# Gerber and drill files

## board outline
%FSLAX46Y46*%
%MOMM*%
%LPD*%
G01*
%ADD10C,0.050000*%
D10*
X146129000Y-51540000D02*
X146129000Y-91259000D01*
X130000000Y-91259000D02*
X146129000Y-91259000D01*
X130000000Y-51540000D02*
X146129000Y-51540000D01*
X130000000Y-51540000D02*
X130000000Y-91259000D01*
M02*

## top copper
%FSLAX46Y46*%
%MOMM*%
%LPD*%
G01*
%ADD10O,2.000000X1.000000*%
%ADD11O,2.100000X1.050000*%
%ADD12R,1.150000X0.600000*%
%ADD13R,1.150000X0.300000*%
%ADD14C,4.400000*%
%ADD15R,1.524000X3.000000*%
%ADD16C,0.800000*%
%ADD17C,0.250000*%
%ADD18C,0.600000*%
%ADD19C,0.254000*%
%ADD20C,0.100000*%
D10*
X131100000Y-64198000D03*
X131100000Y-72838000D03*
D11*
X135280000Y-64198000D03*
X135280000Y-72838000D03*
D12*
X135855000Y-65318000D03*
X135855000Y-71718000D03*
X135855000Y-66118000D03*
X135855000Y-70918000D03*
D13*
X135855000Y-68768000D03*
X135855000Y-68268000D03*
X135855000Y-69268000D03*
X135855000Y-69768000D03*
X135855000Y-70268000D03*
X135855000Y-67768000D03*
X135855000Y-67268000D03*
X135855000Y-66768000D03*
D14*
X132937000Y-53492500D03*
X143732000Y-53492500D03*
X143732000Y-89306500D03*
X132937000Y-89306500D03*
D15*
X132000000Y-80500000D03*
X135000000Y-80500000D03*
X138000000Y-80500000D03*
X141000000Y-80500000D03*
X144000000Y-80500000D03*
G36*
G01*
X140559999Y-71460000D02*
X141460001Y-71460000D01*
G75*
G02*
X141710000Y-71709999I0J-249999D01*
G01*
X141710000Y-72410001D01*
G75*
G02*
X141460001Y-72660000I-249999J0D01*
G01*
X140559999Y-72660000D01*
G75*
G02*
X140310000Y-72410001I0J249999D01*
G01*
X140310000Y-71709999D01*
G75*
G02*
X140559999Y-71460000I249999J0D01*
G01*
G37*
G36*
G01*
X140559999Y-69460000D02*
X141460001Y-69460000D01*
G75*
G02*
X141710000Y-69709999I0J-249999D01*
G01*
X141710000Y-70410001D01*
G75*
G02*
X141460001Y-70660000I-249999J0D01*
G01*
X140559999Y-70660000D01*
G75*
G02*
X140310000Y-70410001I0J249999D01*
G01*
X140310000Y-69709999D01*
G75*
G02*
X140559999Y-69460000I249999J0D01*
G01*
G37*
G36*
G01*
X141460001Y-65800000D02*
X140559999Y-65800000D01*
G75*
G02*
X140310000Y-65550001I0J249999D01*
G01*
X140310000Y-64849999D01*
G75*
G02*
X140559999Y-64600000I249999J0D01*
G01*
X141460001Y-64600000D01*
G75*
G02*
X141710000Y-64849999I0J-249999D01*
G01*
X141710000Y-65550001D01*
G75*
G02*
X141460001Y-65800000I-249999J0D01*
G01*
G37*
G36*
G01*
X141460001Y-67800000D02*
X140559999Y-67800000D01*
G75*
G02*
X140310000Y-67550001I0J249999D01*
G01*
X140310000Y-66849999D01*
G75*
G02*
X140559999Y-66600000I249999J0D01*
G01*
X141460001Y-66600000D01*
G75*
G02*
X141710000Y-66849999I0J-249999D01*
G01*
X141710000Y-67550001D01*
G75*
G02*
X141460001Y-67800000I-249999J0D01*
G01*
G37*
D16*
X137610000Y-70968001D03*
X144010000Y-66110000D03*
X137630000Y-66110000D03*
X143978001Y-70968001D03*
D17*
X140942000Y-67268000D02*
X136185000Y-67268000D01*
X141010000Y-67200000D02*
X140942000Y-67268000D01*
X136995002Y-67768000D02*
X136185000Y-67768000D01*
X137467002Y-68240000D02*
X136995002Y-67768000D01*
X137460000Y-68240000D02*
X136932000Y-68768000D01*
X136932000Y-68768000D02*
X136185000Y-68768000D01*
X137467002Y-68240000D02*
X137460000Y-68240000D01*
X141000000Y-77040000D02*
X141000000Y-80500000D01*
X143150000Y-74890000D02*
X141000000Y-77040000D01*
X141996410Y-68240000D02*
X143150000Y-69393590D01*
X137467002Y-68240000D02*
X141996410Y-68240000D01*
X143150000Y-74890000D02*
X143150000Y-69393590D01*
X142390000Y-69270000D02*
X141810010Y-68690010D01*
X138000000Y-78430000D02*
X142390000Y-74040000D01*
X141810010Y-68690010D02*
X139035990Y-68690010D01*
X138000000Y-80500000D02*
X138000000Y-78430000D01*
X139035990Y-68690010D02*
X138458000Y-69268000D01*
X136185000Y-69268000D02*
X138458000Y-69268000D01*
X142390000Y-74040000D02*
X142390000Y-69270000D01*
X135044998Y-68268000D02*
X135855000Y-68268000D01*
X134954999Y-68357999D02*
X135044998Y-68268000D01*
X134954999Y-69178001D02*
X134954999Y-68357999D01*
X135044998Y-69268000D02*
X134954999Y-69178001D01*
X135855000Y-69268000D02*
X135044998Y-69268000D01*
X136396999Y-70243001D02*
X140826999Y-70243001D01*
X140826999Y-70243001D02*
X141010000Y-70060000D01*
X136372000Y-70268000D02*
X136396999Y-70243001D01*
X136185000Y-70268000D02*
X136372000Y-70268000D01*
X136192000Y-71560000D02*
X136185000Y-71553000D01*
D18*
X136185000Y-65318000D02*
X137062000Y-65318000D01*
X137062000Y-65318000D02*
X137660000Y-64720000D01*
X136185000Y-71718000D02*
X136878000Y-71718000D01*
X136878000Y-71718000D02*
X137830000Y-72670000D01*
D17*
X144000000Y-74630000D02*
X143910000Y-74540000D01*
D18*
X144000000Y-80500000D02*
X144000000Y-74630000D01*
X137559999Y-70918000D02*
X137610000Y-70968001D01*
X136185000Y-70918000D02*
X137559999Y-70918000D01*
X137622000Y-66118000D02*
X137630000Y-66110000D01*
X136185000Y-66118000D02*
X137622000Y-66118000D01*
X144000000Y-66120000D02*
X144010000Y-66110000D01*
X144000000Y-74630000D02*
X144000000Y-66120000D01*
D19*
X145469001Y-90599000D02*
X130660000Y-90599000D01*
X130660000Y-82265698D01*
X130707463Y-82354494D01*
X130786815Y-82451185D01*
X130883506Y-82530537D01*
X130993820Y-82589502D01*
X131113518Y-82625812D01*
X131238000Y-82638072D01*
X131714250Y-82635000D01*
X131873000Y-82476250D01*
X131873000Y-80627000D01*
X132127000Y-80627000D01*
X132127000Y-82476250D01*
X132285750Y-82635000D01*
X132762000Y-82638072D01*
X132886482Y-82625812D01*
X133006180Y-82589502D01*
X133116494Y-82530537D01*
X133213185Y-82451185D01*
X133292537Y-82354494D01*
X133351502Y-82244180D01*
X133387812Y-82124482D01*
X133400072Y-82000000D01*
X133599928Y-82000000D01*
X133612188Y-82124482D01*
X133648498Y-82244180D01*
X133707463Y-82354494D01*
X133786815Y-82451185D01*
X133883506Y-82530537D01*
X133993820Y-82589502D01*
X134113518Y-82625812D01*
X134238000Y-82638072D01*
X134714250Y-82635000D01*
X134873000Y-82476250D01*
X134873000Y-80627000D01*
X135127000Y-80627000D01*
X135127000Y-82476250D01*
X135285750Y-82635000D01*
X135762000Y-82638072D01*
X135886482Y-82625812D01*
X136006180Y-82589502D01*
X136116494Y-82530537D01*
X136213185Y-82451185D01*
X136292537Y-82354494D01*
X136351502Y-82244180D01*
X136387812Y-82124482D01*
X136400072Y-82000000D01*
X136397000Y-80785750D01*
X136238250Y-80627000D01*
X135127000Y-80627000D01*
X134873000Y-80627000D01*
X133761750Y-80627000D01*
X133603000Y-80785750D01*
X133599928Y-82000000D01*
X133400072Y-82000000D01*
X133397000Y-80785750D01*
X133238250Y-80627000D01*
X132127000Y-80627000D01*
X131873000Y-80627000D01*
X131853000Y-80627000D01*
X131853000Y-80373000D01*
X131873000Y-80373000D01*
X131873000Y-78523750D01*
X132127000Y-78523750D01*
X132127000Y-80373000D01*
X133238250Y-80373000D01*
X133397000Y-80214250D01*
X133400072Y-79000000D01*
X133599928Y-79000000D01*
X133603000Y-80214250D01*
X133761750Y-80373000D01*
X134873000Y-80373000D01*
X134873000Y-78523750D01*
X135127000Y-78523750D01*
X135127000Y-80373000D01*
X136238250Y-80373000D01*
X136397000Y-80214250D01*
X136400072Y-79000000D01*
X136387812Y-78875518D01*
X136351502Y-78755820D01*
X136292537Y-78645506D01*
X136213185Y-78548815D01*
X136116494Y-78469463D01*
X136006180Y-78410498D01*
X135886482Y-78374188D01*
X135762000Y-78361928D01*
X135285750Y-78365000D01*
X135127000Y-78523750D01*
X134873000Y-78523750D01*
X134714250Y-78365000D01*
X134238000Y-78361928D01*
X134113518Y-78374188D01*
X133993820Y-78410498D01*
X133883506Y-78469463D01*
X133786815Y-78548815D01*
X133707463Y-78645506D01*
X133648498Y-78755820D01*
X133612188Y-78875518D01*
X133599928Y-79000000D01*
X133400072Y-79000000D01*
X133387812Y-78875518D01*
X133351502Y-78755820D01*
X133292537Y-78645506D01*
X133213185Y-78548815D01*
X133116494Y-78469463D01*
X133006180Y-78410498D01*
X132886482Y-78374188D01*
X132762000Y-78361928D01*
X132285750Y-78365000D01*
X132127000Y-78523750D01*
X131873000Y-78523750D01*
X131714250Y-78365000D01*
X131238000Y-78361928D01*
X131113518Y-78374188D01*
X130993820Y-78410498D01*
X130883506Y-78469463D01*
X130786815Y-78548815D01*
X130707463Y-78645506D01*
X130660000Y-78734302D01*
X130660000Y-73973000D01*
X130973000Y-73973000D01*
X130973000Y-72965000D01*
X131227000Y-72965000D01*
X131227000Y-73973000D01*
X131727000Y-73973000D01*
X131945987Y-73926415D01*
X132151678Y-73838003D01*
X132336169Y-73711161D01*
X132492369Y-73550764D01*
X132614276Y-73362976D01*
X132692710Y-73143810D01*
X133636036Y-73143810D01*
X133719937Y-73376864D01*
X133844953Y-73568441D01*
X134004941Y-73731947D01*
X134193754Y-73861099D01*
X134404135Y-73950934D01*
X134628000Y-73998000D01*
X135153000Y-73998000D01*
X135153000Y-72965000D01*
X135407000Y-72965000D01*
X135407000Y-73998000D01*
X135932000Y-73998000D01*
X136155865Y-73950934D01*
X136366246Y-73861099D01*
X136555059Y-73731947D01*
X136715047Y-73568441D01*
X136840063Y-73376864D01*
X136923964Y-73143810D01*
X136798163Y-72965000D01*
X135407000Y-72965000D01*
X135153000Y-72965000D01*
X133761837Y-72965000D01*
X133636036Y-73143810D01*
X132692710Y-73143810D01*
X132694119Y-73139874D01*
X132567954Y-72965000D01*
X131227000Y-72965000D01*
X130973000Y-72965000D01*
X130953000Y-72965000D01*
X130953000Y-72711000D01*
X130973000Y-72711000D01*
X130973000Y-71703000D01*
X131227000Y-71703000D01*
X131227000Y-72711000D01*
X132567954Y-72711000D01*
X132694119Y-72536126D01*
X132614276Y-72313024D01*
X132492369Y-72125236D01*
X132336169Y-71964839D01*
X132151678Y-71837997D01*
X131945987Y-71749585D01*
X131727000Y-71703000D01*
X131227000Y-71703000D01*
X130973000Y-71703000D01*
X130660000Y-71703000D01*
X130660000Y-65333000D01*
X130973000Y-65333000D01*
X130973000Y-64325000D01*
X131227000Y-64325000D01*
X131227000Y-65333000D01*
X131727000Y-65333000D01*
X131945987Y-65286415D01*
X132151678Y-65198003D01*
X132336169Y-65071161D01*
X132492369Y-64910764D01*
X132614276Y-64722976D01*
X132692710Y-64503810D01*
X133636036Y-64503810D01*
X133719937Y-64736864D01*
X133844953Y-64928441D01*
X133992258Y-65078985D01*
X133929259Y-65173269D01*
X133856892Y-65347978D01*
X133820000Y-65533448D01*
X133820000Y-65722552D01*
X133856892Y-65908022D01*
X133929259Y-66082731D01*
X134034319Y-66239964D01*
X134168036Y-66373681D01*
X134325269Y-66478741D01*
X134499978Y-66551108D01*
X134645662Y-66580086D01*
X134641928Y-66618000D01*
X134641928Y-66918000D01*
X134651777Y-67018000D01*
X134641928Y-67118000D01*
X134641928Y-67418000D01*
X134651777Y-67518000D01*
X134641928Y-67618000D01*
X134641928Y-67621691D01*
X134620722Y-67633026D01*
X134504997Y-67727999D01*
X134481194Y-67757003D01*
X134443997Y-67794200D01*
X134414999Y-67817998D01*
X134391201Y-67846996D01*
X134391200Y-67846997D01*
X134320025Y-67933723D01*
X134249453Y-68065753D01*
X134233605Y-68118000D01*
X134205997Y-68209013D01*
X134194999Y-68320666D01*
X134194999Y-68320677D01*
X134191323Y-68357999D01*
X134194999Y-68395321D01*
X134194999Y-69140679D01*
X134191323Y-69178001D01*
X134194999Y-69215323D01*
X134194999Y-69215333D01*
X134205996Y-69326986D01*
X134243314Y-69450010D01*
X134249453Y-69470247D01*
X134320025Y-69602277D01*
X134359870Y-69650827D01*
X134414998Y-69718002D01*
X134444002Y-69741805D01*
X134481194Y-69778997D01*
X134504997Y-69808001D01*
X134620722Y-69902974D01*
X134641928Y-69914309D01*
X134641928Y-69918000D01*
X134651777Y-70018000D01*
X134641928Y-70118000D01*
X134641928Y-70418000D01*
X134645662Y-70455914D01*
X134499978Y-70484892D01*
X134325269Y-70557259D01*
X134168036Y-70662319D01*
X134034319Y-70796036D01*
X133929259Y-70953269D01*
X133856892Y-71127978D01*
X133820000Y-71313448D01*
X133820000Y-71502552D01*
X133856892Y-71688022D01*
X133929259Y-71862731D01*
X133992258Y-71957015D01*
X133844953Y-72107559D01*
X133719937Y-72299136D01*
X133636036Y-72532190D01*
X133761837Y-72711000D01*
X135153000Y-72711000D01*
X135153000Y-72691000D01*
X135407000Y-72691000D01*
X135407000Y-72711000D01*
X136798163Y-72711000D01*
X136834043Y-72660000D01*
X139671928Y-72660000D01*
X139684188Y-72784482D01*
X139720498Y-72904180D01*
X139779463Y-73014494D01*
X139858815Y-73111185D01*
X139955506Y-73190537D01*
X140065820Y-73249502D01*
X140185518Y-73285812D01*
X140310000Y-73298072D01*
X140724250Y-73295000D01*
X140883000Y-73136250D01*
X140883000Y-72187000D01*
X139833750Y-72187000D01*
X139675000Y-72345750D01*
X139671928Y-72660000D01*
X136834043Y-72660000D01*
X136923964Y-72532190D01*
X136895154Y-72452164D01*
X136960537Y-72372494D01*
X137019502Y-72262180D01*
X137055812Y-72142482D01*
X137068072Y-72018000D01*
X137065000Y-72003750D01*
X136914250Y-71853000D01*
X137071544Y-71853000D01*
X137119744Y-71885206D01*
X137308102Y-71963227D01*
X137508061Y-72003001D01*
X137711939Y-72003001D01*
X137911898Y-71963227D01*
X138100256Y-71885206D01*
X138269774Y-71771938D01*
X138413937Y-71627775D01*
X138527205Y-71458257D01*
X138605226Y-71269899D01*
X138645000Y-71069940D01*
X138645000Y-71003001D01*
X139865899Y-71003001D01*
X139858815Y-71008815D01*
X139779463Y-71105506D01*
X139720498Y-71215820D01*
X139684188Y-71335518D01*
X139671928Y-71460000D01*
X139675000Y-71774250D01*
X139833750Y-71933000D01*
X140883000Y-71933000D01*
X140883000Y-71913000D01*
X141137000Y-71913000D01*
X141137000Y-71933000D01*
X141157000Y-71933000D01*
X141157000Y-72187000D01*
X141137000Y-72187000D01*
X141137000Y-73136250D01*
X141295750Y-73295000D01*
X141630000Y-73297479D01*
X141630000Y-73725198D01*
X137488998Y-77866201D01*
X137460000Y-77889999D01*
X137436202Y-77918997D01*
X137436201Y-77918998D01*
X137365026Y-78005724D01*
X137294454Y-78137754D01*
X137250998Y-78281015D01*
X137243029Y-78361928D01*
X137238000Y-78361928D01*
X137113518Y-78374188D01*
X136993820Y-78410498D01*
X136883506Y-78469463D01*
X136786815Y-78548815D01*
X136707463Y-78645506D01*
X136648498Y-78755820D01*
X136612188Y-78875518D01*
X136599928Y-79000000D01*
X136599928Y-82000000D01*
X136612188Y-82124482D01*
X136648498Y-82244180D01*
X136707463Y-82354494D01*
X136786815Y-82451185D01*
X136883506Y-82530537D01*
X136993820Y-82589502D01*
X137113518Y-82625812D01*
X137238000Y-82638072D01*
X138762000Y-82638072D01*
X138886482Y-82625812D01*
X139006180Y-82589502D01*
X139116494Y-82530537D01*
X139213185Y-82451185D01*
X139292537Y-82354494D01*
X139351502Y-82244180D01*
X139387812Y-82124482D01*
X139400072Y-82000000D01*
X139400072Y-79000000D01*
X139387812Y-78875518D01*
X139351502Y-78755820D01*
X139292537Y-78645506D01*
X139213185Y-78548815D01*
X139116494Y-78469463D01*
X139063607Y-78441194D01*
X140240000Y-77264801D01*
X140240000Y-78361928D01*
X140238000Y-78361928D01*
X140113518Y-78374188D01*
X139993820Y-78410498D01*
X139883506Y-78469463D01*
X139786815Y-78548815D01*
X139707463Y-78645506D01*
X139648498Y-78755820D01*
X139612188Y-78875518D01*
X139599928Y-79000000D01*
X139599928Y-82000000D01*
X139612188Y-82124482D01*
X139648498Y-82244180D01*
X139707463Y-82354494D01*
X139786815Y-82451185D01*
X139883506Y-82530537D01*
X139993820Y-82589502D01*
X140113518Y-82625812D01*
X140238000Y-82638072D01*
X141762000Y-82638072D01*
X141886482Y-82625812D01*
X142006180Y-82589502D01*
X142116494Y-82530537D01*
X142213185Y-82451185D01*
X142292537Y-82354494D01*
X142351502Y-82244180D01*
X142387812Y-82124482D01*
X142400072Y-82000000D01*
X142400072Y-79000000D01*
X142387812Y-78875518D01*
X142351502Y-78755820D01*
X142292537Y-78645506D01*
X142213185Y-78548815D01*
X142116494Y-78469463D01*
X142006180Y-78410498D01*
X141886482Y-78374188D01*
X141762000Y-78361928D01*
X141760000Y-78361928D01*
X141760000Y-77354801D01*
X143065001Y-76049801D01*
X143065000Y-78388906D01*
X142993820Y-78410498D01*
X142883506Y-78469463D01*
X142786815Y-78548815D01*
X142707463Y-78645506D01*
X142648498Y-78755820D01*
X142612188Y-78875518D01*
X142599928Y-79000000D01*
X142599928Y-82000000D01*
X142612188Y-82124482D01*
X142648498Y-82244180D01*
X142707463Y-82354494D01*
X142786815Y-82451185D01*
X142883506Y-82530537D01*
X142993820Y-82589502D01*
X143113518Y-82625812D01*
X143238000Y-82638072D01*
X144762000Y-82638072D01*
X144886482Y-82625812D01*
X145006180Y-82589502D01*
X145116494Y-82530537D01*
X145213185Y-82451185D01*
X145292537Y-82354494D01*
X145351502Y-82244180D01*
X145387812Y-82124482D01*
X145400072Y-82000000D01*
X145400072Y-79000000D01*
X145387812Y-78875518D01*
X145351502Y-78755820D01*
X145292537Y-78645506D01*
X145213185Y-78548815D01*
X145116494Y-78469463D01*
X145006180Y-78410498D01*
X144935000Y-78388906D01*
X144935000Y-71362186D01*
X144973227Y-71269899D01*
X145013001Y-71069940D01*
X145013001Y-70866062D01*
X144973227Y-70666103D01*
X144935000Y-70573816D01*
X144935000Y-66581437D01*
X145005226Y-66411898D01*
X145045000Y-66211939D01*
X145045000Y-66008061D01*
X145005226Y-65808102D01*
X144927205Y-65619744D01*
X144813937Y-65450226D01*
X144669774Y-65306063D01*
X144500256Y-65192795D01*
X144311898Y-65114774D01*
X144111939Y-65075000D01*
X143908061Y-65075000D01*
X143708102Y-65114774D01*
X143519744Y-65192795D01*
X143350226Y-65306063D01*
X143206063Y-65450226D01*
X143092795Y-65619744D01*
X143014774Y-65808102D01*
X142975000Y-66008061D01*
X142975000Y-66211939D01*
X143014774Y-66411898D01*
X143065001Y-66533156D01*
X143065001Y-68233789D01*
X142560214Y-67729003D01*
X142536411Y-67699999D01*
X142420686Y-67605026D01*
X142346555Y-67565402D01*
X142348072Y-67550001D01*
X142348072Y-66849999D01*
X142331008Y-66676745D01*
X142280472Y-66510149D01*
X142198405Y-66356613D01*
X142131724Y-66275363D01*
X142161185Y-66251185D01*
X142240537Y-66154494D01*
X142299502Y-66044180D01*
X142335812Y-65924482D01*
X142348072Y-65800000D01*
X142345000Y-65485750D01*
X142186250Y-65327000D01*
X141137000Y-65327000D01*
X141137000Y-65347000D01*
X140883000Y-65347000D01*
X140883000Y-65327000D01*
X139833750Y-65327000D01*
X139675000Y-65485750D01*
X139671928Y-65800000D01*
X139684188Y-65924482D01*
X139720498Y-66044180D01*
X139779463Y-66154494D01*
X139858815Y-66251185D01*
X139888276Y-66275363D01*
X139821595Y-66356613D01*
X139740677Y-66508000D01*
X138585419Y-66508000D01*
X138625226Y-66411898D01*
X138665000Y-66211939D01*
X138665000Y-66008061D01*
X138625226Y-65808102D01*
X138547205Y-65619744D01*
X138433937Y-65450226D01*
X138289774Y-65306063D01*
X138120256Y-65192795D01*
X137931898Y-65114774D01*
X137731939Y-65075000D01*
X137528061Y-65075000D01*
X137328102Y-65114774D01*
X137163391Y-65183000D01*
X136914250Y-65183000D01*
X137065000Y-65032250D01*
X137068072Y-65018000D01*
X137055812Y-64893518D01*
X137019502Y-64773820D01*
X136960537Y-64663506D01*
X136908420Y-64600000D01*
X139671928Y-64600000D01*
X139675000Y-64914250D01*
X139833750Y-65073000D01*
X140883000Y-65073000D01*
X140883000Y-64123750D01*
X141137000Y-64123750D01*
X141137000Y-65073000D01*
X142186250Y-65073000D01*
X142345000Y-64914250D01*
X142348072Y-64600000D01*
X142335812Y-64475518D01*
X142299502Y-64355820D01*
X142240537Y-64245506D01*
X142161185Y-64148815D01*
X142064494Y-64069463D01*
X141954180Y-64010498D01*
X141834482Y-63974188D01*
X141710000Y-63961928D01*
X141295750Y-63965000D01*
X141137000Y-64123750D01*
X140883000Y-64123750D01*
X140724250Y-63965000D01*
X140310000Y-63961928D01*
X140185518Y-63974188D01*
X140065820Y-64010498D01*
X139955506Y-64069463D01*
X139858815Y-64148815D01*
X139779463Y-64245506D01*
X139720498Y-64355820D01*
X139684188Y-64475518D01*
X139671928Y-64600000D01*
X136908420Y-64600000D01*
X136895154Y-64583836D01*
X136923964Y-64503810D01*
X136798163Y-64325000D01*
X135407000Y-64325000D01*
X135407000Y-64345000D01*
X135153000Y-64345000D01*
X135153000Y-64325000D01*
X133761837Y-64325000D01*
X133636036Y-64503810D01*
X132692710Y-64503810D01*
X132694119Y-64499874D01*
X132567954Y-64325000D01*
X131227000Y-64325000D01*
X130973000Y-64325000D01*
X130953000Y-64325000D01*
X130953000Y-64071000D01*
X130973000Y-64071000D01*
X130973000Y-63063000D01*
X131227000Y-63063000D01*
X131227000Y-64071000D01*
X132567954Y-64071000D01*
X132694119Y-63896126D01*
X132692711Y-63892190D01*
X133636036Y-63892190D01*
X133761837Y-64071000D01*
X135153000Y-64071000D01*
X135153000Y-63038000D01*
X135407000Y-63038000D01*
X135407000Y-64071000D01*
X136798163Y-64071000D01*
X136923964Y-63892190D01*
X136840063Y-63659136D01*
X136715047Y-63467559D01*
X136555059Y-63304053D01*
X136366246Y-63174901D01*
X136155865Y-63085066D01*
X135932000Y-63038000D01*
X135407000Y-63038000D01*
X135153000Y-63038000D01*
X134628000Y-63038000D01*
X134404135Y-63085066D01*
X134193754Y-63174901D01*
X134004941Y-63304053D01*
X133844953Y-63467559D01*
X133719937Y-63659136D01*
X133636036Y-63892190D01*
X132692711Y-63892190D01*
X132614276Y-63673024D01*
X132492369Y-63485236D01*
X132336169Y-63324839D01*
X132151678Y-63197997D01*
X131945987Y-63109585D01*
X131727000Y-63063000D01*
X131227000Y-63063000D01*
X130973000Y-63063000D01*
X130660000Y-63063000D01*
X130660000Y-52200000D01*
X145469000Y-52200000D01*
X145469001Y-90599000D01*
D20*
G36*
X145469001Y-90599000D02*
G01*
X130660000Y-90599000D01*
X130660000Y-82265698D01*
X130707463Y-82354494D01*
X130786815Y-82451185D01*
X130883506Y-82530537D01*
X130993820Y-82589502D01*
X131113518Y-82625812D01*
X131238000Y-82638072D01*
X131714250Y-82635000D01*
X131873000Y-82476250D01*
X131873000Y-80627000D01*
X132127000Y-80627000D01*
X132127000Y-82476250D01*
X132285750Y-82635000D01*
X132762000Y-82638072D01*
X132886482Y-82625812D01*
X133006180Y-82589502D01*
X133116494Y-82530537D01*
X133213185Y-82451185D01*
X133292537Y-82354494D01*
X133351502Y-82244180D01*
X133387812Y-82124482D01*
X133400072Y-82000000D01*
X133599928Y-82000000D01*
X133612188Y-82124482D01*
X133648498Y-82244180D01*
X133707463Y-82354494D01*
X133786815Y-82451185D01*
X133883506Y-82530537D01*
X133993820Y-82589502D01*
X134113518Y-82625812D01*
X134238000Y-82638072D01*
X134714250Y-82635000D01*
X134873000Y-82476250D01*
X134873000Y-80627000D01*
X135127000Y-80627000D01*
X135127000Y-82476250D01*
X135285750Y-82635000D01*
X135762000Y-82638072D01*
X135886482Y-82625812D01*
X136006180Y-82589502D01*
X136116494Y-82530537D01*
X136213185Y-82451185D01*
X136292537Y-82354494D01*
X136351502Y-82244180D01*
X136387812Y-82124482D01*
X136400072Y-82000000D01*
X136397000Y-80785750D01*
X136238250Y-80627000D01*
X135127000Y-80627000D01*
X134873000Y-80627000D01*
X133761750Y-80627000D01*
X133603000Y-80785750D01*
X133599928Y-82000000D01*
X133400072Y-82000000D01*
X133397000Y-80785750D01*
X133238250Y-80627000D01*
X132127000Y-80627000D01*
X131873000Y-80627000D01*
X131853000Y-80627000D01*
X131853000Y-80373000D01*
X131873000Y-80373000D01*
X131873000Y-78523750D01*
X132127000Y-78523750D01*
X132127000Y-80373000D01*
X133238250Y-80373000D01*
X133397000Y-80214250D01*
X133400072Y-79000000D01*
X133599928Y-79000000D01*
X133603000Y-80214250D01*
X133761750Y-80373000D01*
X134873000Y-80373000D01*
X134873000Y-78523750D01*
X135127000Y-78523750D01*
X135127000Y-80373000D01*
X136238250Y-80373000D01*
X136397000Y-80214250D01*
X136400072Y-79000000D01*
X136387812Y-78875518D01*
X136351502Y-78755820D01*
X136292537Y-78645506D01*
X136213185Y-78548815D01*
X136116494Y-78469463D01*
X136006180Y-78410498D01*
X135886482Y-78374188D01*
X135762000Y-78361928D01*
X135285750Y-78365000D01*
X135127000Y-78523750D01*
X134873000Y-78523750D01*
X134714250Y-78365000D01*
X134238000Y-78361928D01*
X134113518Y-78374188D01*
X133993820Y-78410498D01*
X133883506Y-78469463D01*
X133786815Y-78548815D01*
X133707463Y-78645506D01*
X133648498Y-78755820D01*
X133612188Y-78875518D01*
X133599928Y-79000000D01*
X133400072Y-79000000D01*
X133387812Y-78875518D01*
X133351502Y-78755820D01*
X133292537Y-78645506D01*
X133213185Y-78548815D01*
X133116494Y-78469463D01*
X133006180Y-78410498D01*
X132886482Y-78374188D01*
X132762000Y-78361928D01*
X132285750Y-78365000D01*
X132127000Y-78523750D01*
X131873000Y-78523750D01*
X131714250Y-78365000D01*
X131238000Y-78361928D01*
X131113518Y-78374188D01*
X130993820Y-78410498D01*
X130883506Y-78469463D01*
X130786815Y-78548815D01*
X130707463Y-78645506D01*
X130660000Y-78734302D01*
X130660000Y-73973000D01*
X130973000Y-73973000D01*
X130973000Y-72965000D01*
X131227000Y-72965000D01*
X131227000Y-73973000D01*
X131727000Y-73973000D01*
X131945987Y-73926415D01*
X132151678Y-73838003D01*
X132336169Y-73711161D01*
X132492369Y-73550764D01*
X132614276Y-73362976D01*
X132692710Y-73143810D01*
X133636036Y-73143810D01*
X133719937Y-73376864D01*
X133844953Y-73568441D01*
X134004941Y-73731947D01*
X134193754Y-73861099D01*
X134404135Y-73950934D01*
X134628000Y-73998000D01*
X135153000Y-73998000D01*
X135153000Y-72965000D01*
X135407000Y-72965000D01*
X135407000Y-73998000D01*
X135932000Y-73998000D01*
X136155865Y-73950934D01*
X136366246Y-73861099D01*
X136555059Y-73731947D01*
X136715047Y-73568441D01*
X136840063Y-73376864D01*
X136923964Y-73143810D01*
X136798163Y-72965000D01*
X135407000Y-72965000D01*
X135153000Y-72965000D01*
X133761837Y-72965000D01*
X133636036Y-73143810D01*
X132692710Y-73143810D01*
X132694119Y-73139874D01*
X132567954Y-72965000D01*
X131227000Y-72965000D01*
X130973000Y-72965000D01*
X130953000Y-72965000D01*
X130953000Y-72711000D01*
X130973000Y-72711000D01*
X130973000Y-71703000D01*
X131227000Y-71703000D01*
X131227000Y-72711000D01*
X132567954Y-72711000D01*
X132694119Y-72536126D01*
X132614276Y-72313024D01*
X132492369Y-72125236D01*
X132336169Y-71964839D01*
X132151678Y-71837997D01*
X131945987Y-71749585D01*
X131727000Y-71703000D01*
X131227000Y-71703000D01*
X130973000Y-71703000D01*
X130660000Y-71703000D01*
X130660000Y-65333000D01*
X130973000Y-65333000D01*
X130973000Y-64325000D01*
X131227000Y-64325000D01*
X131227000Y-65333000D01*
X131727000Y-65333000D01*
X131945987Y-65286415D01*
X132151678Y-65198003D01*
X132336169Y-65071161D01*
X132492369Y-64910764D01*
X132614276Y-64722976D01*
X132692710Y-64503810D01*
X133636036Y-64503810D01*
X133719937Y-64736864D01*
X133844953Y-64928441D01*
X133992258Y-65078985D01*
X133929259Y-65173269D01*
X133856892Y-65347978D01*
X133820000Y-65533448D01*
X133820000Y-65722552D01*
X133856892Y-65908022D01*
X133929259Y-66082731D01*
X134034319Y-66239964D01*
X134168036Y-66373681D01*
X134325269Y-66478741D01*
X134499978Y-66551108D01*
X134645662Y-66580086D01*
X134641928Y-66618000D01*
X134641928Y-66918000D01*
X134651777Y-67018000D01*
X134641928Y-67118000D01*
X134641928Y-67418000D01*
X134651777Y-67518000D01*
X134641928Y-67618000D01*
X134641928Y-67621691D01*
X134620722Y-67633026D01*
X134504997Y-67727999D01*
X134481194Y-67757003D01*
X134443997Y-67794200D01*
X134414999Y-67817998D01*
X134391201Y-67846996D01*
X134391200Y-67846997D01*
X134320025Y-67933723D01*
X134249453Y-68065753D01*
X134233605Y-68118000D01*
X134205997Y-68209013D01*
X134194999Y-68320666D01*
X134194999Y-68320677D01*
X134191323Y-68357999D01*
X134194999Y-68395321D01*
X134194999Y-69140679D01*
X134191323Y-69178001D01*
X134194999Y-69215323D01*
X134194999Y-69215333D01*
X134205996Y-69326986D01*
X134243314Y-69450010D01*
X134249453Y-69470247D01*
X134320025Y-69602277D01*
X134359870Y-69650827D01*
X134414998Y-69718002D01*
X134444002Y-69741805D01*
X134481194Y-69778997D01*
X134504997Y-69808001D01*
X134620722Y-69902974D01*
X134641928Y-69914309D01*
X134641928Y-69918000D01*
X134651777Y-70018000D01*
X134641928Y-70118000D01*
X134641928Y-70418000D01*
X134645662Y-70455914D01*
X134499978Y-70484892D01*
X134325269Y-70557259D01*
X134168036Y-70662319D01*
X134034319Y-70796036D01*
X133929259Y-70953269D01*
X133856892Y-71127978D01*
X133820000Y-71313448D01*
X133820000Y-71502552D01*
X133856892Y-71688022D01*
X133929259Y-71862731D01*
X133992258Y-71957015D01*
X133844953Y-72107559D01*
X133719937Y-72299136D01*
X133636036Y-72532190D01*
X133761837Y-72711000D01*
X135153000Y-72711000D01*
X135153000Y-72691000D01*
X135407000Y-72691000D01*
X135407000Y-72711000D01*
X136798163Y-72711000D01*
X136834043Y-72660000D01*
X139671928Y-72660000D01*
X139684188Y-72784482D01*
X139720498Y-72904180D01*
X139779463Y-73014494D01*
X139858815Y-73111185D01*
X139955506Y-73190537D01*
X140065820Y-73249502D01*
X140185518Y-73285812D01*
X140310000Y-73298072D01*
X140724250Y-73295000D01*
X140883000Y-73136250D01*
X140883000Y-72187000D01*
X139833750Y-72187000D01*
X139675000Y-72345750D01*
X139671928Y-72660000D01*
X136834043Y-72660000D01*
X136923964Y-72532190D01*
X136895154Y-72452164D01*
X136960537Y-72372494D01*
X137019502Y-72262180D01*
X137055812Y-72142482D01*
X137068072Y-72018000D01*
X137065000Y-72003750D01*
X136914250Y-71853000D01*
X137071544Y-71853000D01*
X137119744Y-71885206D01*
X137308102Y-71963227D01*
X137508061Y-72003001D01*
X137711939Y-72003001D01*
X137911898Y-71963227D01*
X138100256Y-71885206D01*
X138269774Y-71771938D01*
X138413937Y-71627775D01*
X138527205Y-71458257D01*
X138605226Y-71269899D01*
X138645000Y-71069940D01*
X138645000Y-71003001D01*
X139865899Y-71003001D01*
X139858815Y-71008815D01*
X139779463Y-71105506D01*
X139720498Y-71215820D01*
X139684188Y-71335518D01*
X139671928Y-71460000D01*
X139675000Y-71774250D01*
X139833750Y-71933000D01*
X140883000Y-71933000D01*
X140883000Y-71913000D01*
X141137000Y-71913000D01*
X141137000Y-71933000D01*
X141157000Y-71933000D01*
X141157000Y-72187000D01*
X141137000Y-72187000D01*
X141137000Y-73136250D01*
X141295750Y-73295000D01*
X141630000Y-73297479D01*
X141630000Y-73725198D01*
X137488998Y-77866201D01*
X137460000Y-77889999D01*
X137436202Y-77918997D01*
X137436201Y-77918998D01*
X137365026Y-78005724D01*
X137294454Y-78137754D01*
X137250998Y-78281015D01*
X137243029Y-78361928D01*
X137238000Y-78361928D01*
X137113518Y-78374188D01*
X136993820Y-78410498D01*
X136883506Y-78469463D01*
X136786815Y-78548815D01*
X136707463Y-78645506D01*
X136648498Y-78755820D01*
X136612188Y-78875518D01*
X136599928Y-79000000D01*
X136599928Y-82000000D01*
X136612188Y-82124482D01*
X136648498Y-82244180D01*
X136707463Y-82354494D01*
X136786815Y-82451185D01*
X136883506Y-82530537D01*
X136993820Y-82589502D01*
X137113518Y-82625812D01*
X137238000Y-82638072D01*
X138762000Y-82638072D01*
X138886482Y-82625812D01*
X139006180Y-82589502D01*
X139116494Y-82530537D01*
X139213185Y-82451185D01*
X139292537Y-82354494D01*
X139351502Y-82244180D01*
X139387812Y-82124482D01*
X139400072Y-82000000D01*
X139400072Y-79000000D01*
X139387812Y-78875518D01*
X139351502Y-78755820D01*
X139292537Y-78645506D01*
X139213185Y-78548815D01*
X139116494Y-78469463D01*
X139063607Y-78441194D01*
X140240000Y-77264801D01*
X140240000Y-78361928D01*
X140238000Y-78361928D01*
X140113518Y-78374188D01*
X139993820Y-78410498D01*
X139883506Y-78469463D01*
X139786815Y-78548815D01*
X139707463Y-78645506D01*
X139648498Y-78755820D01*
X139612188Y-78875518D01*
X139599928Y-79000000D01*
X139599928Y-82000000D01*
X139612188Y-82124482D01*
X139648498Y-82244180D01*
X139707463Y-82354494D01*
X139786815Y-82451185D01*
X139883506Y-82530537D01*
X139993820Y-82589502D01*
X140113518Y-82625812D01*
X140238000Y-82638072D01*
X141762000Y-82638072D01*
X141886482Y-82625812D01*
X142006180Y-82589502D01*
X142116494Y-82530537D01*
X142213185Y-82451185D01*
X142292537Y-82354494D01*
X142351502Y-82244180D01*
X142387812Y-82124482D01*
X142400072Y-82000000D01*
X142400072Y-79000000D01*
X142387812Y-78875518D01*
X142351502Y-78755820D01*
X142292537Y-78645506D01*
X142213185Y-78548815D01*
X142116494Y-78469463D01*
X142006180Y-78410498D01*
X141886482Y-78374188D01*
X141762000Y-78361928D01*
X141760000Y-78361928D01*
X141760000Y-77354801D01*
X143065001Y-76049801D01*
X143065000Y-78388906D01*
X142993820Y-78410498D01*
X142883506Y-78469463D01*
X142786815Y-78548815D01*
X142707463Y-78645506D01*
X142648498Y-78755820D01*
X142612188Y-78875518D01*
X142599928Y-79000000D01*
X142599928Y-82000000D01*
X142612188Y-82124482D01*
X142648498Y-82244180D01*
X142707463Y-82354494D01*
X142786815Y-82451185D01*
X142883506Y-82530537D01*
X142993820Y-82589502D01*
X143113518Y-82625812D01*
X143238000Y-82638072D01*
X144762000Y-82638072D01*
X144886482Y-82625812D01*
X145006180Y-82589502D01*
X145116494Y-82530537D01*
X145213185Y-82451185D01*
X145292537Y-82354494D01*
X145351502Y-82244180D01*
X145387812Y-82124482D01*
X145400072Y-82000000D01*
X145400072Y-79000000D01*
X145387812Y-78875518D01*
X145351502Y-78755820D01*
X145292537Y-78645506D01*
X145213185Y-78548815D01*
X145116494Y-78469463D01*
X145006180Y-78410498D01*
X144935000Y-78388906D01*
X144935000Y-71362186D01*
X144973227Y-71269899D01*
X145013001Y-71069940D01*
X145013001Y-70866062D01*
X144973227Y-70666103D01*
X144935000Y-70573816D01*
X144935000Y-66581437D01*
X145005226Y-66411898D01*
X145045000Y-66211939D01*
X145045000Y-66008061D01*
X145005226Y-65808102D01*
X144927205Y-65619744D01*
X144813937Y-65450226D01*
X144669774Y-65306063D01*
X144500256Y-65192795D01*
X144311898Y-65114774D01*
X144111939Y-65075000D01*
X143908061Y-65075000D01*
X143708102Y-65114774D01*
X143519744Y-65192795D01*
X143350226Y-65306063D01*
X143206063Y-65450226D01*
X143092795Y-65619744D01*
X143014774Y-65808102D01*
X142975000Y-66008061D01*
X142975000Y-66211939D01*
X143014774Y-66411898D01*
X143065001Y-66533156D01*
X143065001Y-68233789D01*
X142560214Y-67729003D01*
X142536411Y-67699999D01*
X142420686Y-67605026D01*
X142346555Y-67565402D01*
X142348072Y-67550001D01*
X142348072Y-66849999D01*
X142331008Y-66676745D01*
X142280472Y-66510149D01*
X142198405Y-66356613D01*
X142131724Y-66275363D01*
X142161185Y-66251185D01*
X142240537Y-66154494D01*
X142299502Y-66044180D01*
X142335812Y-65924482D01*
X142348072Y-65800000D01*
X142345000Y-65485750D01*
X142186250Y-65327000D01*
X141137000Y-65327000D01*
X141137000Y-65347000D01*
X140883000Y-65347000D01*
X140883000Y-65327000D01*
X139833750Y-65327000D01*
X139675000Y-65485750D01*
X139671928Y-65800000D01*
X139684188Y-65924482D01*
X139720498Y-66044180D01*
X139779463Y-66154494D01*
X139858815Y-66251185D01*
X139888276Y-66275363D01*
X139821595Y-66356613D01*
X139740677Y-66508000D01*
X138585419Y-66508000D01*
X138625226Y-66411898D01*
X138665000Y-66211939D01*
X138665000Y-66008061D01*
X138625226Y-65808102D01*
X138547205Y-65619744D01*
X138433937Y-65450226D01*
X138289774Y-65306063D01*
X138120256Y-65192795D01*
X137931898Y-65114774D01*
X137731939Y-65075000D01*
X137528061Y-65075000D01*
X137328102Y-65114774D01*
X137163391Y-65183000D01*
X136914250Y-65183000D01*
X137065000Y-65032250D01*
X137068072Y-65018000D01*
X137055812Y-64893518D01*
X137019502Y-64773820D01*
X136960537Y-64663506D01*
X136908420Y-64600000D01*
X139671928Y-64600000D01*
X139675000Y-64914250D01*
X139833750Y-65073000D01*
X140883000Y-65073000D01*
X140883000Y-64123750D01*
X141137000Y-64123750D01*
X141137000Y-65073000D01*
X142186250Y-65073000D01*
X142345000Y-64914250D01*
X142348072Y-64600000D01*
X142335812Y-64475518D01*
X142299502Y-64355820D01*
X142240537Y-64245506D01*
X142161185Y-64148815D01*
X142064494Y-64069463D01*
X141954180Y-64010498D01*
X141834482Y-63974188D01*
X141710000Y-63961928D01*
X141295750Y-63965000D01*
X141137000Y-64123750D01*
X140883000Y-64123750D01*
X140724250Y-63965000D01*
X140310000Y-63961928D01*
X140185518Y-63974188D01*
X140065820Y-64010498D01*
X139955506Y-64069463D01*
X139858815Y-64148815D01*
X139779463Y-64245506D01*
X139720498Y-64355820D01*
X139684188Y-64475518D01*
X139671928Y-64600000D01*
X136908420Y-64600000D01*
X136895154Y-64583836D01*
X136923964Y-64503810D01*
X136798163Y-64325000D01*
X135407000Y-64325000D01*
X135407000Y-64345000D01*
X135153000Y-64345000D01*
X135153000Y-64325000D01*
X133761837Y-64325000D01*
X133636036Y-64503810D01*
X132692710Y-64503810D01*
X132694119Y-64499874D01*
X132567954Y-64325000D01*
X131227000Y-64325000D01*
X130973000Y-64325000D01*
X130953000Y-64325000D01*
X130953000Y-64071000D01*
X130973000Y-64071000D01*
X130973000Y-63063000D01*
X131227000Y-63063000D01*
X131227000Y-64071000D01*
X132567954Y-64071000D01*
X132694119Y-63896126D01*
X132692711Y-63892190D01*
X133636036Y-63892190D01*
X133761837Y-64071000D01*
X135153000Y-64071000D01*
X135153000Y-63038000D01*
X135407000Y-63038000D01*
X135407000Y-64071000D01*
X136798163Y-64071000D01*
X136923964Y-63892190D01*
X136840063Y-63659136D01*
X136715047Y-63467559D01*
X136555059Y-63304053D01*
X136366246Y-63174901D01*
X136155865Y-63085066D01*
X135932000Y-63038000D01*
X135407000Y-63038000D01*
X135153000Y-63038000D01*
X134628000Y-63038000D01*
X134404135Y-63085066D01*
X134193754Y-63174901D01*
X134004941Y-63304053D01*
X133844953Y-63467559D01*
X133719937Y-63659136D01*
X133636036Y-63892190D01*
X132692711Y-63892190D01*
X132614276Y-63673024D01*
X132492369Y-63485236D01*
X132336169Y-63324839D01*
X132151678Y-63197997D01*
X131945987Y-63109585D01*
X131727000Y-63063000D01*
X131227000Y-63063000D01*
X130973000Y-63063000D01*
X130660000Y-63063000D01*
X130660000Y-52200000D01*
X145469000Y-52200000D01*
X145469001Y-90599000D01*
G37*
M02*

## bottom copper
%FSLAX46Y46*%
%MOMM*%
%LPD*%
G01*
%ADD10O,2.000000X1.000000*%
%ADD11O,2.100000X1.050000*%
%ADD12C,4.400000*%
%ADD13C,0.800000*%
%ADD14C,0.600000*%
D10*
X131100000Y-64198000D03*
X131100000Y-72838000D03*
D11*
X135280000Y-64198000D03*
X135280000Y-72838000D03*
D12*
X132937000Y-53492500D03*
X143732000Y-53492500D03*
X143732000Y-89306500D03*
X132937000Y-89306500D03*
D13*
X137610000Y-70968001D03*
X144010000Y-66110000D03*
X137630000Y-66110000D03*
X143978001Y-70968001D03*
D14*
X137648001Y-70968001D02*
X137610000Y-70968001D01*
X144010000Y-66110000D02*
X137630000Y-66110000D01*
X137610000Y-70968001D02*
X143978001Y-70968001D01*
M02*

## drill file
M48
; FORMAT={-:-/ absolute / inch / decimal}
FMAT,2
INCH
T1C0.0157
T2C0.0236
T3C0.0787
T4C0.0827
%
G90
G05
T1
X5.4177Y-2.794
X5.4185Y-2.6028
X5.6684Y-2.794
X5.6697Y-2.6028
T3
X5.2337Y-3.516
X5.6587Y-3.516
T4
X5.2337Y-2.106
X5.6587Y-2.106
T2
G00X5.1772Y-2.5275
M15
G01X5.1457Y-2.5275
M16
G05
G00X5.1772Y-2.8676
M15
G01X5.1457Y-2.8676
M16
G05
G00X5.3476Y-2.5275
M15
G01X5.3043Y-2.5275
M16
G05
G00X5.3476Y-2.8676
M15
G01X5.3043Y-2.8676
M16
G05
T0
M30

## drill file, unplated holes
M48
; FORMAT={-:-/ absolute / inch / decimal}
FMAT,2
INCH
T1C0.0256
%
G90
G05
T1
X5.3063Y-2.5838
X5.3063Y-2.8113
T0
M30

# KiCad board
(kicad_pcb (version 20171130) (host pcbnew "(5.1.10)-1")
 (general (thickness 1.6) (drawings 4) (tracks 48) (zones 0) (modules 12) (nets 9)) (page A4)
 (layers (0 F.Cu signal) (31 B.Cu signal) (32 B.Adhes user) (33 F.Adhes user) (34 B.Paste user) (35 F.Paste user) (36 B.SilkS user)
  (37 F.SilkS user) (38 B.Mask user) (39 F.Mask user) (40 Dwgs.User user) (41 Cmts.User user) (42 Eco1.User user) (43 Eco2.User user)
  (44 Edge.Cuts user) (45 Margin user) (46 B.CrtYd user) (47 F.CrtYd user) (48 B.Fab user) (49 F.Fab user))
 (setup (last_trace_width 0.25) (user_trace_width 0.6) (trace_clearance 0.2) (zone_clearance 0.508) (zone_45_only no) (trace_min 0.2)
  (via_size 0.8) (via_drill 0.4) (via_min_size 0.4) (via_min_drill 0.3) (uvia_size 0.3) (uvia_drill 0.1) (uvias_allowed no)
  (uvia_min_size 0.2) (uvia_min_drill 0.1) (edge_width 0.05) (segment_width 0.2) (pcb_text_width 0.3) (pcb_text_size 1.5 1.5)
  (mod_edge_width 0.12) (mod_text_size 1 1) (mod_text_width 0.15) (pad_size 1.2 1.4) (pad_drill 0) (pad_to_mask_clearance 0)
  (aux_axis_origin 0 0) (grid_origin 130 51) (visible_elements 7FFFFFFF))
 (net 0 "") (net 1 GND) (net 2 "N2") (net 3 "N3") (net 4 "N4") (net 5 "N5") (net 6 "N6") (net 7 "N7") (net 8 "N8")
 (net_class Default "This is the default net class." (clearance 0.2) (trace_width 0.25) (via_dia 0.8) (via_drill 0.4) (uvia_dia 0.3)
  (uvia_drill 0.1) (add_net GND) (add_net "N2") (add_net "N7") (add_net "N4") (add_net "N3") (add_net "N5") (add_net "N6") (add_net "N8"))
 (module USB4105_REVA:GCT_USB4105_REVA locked (layer F.Cu) (at 131.1 68.518 270)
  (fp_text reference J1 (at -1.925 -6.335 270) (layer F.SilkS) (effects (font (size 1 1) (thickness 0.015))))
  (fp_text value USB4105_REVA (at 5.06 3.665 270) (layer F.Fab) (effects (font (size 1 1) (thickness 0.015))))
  (pad G1 thru_hole oval (at -4.32 0 270) (size 1 2) (drill oval 0.6 1.4) (layers *.Cu *.Mask) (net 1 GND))
  (pad G2 thru_hole oval (at 4.32 0 270) (size 1 2) (drill oval 0.6 1.4) (layers *.Cu *.Mask) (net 1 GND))
  (pad G3 thru_hole oval (at -4.32 -4.18 270) (size 1.05 2.1) (drill oval 0.6 1.7) (layers *.Cu *.Mask) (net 1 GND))
  (pad G4 thru_hole oval (at 4.32 -4.18 270) (size 1.05 2.1) (drill oval 0.6 1.7) (layers *.Cu *.Mask) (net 1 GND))
  (pad None np_thru_hole circle (at 2.89 -3.68 270) (size 0.65 0.65) (drill 0.65) (layers *.Cu *.Mask))
  (pad None np_thru_hole circle (at -2.89 -3.68 270) (size 0.65 0.65) (drill 0.65) (layers *.Cu *.Mask))
  (pad A1/B12 smd rect (at -3.2 -4.755 270) (size 0.6 1.15) (layers F.Cu F.Paste F.Mask) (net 1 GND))
  (pad B1/A12 smd rect (at 3.2 -4.755 270) (size 0.6 1.15) (layers F.Cu F.Paste F.Mask) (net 1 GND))
  (pad A4/B9 smd rect (at -2.4 -4.755 270) (size 0.6 1.15) (layers F.Cu F.Paste F.Mask) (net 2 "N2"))
  (pad B4/A9 smd rect (at 2.4 -4.755 270) (size 0.6 1.15) (layers F.Cu F.Paste F.Mask) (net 2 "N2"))
  (pad A7 smd rect (at 0.25 -4.755 270) (size 0.3 1.15) (layers F.Cu F.Paste F.Mask) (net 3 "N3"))
  (pad A6 smd rect (at -0.25 -4.755 270) (size 0.3 1.15) (layers F.Cu F.Paste F.Mask) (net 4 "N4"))
  (pad B6 smd rect (at 0.75 -4.755 270) (size 0.3 1.15) (layers F.Cu F.Paste F.Mask) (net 4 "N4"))
  (pad A8 smd rect (at 1.25 -4.755 270) (size 0.3 1.15) (layers F.Cu F.Paste F.Mask) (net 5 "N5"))
  (pad B5 smd rect (at 1.75 -4.755 270) (size 0.3 1.15) (layers F.Cu F.Paste F.Mask) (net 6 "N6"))
  (pad B7 smd rect (at -0.75 -4.755 270) (size 0.3 1.15) (layers F.Cu F.Paste F.Mask) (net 3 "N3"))
  (pad A5 smd rect (at -1.25 -4.755 270) (size 0.3 1.15) (layers F.Cu F.Paste F.Mask) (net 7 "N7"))
  (pad B8 smd rect (at -1.75 -4.755 270) (size 0.3 1.15) (layers F.Cu F.Paste F.Mask) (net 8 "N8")))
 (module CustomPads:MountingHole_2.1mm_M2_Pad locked (layer F.Cu) (at 132.937 53.4925) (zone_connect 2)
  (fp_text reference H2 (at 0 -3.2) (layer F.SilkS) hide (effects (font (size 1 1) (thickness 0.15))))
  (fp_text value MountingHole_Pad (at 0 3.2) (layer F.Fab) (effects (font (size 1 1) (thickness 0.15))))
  (pad 1 thru_hole circle (at 0 0) (size 4.4 4.4) (drill 2.1) (layers *.Cu *.Mask) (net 1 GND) (zone_connect 2)))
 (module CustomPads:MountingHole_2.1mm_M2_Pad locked (layer F.Cu) (at 143.732 53.4925) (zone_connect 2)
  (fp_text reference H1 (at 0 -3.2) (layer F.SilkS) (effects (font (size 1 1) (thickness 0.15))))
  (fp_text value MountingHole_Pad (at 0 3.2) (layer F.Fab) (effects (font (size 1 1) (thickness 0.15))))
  (pad 1 thru_hole circle (at 0 0) (size 4.4 4.4) (drill 2.1) (layers *.Cu *.Mask) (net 1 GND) (zone_connect 2)))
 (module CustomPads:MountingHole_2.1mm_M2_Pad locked (layer F.Cu) (at 143.732 89.3065) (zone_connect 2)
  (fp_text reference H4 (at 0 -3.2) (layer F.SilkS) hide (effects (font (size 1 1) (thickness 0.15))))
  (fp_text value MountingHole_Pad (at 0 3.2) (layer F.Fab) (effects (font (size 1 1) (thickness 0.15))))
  (pad 1 thru_hole circle (at 0 0) (size 4.4 4.4) (drill 2) (layers *.Cu *.Mask) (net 1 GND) (zone_connect 2)))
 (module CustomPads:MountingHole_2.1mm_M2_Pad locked (layer F.Cu) (at 132.937 89.3065) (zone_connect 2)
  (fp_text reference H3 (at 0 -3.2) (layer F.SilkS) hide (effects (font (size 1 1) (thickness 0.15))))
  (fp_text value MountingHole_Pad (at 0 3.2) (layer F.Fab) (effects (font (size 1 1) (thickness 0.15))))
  (pad 1 thru_hole circle (at 0 0) (size 4.4 4.4) (drill 2) (layers *.Cu *.Mask) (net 1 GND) (zone_connect 2)))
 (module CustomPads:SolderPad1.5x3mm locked (layer F.Cu) (at 130 79.5 90)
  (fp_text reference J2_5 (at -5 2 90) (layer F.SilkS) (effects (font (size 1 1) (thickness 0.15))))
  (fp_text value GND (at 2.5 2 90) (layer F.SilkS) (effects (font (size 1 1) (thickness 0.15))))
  (pad 1 smd rect (at -1 2 90) (size 3 1.524) (layers F.Cu F.Paste F.Mask) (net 1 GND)))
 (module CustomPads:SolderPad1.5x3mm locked (layer F.Cu) (at 133 79.5 90)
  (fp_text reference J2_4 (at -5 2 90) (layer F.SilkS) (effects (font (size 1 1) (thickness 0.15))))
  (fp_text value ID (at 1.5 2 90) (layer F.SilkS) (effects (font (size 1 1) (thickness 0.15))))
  (pad 1 smd rect (at -1 2 90) (size 3 1.524) (layers F.Cu F.Paste F.Mask) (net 1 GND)))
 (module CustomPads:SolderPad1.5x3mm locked (layer F.Cu) (at 140 81.5 270)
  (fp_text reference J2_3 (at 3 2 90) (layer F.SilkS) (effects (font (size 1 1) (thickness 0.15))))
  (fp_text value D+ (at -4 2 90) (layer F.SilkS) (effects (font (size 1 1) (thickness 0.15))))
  (pad 1 smd rect (at -1 2 270) (size 3 1.524) (layers F.Cu F.Paste F.Mask) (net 4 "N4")))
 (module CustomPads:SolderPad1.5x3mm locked (layer F.Cu) (at 139 79.5 90)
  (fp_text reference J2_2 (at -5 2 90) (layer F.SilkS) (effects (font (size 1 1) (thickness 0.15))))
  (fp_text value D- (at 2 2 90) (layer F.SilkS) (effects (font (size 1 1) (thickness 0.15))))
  (pad 1 smd rect (at -1 2 90) (size 3 1.524) (layers F.Cu F.Paste F.Mask) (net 3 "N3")))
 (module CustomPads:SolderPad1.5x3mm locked (layer F.Cu) (at 146 81.5 270)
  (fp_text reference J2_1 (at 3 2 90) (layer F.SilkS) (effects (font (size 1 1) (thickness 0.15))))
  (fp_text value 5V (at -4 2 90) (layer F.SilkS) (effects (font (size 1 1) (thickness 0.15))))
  (pad 1 smd rect (at -1 2 270) (size 3 1.524) (layers F.Cu F.Paste F.Mask) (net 2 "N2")))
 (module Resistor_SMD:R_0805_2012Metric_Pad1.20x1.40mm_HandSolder (layer F.Cu) (at 141.01 71.06 270)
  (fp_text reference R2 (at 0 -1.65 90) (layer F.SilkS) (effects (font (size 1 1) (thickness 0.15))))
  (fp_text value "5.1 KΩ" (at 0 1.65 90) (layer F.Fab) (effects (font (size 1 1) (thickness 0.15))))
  (pad 2 smd roundrect (at 1 0 270) (size 1.2 1.4) (layers F.Cu F.Paste F.Mask) (roundrect_rratio 0.2083325) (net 1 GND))
  (pad 1 smd roundrect (at -1 0 270) (size 1.2 1.4) (layers F.Cu F.Paste F.Mask) (roundrect_rratio 0.2083325) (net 6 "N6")))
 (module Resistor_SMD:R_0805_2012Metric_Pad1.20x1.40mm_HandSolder (layer F.Cu) (at 141.01 66.2 90)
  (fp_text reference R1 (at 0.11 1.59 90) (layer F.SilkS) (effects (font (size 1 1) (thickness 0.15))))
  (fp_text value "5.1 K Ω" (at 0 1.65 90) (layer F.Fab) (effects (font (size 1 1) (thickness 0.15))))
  (pad 2 smd roundrect (at 1 0 90) (size 1.2 1.4) (layers F.Cu F.Paste F.Mask) (roundrect_rratio 0.2083325) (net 1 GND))
  (pad 1 smd roundrect (at -1 0 90) (size 1.2 1.4) (layers F.Cu F.Paste F.Mask) (roundrect_rratio 0.2083325) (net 7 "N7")))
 (gr_line (start 146.129 51.54) (end 146.129 91.259) (layer Edge.Cuts) (width 0.05))
 (gr_line (start 130 91.259) (end 146.129 91.259) (layer Edge.Cuts) (width 0.05))
 (gr_line (start 130 51.54) (end 146.129 51.54) (layer Edge.Cuts) (width 0.05))
 (gr_line (start 130 51.54) (end 130 91.259) (layer Edge.Cuts) (width 0.05))
 (segment (start 140.942 67.268) (end 136.185 67.268) (width 0.25) (layer F.Cu) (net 7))
 (segment (start 141.01 67.2) (end 140.942 67.268) (width 0.25) (layer F.Cu) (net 7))
 (segment (start 136.995002 67.768) (end 136.185 67.768) (width 0.25) (layer F.Cu) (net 3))
 (segment (start 137.467002 68.24) (end 136.995002 67.768) (width 0.25) (layer F.Cu) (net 3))
 (segment (start 137.46 68.24) (end 136.932 68.768) (width 0.25) (layer F.Cu) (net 3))
 (segment (start 136.932 68.768) (end 136.185 68.768) (width 0.25) (layer F.Cu) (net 3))
 (segment (start 137.467002 68.24) (end 137.46 68.24) (width 0.25) (layer F.Cu) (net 3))
 (segment (start 141 77.04) (end 141 80.5) (width 0.25) (layer F.Cu) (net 3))
 (segment (start 143.15 74.89) (end 141 77.04) (width 0.25) (layer F.Cu) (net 3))
 (segment (start 141.99641 68.24) (end 143.15 69.39359) (width 0.25) (layer F.Cu) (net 3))
 (segment (start 137.467002 68.24) (end 141.99641 68.24) (width 0.25) (layer F.Cu) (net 3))
 (segment (start 143.15 74.89) (end 143.15 69.39359) (width 0.25) (layer F.Cu) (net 3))
 (segment (start 142.39 69.27) (end 141.81001 68.69001) (width 0.25) (layer F.Cu) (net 4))
 (segment (start 138 78.43) (end 142.39 74.04) (width 0.25) (layer F.Cu) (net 4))
 (segment (start 141.81001 68.69001) (end 139.03599 68.69001) (width 0.25) (layer F.Cu) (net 4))
 (segment (start 138 80.5) (end 138 78.43) (width 0.25) (layer F.Cu) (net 4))
 (segment (start 139.03599 68.69001) (end 138.458 69.268) (width 0.25) (layer F.Cu) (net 4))
 (segment (start 136.185 69.268) (end 138.458 69.268) (width 0.25) (layer F.Cu) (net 4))
 (segment (start 142.39 74.04) (end 142.39 69.27) (width 0.25) (layer F.Cu) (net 4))
 (segment (start 135.044998 68.268) (end 135.855 68.268) (width 0.25) (layer F.Cu) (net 4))
 (segment (start 134.954999 68.357999) (end 135.044998 68.268) (width 0.25) (layer F.Cu) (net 4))
 (segment (start 134.954999 69.178001) (end 134.954999 68.357999) (width 0.25) (layer F.Cu) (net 4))
 (segment (start 135.044998 69.268) (end 134.954999 69.178001) (width 0.25) (layer F.Cu) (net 4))
 (segment (start 135.855 69.268) (end 135.044998 69.268) (width 0.25) (layer F.Cu) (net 4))
 (segment (start 136.396999 70.243001) (end 140.826999 70.243001) (width 0.25) (layer F.Cu) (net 6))
 (segment (start 140.826999 70.243001) (end 141.01 70.06) (width 0.25) (layer F.Cu) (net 6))
 (segment (start 136.372 70.268) (end 136.396999 70.243001) (width 0.25) (layer F.Cu) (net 6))
 (segment (start 136.185 70.268) (end 136.372 70.268) (width 0.25) (layer F.Cu) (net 6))
 (segment (start 136.192 71.56) (end 136.185 71.553) (width 0.25) (layer F.Cu) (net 1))
 (segment (start 136.185 65.318) (end 137.062 65.318) (width 0.6) (layer F.Cu) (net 1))
 (segment (start 137.062 65.318) (end 137.66 64.72) (width 0.6) (layer F.Cu) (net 1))
 (segment (start 136.185 71.718) (end 136.878 71.718) (width 0.6) (layer F.Cu) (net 1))
 (segment (start 136.878 71.718) (end 137.83 72.67) (width 0.6) (layer F.Cu) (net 1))
 (segment (start 144 74.63) (end 143.91 74.54) (width 0.25) (layer F.Cu) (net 2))
 (segment (start 144 80.5) (end 144 74.63) (width 0.6) (layer F.Cu) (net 2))
 (via (at 137.61 70.968001) (size 0.8) (drill 0.4) (layers F.Cu B.Cu) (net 2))
 (segment (start 137.648001 70.968001) (end 137.61 70.968001) (width 0.6) (layer B.Cu) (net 2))
 (segment (start 137.559999 70.918) (end 137.61 70.968001) (width 0.6) (layer F.Cu) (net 2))
 (segment (start 136.185 70.918) (end 137.559999 70.918) (width 0.6) (layer F.Cu) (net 2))
 (via (at 144.01 66.11) (size 0.8) (drill 0.4) (layers F.Cu B.Cu) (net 2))
 (segment (start 144.01 66.11) (end 137.63 66.11) (width 0.6) (layer B.Cu) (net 2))
 (via (at 137.63 66.11) (size 0.8) (drill 0.4) (layers F.Cu B.Cu) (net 2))
 (segment (start 137.622 66.118) (end 137.63 66.11) (width 0.6) (layer F.Cu) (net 2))
 (segment (start 136.185 66.118) (end 137.622 66.118) (width 0.6) (layer F.Cu) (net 2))
 (segment (start 137.61 70.968001) (end 143.978001 70.968001) (width 0.6) (layer B.Cu) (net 2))
 (via (at 143.978001 70.968001) (size 0.8) (drill 0.4) (layers F.Cu B.Cu) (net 2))
 (segment (start 144 66.12) (end 144.01 66.11) (width 0.6) (layer F.Cu) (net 2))
 (segment (start 144 74.63) (end 144 66.12) (width 0.6) (layer F.Cu) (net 2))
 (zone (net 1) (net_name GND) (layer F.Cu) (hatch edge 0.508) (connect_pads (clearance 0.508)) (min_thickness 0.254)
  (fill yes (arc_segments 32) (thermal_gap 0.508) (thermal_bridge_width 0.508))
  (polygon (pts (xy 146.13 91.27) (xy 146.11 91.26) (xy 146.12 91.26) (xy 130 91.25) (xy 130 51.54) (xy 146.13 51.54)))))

